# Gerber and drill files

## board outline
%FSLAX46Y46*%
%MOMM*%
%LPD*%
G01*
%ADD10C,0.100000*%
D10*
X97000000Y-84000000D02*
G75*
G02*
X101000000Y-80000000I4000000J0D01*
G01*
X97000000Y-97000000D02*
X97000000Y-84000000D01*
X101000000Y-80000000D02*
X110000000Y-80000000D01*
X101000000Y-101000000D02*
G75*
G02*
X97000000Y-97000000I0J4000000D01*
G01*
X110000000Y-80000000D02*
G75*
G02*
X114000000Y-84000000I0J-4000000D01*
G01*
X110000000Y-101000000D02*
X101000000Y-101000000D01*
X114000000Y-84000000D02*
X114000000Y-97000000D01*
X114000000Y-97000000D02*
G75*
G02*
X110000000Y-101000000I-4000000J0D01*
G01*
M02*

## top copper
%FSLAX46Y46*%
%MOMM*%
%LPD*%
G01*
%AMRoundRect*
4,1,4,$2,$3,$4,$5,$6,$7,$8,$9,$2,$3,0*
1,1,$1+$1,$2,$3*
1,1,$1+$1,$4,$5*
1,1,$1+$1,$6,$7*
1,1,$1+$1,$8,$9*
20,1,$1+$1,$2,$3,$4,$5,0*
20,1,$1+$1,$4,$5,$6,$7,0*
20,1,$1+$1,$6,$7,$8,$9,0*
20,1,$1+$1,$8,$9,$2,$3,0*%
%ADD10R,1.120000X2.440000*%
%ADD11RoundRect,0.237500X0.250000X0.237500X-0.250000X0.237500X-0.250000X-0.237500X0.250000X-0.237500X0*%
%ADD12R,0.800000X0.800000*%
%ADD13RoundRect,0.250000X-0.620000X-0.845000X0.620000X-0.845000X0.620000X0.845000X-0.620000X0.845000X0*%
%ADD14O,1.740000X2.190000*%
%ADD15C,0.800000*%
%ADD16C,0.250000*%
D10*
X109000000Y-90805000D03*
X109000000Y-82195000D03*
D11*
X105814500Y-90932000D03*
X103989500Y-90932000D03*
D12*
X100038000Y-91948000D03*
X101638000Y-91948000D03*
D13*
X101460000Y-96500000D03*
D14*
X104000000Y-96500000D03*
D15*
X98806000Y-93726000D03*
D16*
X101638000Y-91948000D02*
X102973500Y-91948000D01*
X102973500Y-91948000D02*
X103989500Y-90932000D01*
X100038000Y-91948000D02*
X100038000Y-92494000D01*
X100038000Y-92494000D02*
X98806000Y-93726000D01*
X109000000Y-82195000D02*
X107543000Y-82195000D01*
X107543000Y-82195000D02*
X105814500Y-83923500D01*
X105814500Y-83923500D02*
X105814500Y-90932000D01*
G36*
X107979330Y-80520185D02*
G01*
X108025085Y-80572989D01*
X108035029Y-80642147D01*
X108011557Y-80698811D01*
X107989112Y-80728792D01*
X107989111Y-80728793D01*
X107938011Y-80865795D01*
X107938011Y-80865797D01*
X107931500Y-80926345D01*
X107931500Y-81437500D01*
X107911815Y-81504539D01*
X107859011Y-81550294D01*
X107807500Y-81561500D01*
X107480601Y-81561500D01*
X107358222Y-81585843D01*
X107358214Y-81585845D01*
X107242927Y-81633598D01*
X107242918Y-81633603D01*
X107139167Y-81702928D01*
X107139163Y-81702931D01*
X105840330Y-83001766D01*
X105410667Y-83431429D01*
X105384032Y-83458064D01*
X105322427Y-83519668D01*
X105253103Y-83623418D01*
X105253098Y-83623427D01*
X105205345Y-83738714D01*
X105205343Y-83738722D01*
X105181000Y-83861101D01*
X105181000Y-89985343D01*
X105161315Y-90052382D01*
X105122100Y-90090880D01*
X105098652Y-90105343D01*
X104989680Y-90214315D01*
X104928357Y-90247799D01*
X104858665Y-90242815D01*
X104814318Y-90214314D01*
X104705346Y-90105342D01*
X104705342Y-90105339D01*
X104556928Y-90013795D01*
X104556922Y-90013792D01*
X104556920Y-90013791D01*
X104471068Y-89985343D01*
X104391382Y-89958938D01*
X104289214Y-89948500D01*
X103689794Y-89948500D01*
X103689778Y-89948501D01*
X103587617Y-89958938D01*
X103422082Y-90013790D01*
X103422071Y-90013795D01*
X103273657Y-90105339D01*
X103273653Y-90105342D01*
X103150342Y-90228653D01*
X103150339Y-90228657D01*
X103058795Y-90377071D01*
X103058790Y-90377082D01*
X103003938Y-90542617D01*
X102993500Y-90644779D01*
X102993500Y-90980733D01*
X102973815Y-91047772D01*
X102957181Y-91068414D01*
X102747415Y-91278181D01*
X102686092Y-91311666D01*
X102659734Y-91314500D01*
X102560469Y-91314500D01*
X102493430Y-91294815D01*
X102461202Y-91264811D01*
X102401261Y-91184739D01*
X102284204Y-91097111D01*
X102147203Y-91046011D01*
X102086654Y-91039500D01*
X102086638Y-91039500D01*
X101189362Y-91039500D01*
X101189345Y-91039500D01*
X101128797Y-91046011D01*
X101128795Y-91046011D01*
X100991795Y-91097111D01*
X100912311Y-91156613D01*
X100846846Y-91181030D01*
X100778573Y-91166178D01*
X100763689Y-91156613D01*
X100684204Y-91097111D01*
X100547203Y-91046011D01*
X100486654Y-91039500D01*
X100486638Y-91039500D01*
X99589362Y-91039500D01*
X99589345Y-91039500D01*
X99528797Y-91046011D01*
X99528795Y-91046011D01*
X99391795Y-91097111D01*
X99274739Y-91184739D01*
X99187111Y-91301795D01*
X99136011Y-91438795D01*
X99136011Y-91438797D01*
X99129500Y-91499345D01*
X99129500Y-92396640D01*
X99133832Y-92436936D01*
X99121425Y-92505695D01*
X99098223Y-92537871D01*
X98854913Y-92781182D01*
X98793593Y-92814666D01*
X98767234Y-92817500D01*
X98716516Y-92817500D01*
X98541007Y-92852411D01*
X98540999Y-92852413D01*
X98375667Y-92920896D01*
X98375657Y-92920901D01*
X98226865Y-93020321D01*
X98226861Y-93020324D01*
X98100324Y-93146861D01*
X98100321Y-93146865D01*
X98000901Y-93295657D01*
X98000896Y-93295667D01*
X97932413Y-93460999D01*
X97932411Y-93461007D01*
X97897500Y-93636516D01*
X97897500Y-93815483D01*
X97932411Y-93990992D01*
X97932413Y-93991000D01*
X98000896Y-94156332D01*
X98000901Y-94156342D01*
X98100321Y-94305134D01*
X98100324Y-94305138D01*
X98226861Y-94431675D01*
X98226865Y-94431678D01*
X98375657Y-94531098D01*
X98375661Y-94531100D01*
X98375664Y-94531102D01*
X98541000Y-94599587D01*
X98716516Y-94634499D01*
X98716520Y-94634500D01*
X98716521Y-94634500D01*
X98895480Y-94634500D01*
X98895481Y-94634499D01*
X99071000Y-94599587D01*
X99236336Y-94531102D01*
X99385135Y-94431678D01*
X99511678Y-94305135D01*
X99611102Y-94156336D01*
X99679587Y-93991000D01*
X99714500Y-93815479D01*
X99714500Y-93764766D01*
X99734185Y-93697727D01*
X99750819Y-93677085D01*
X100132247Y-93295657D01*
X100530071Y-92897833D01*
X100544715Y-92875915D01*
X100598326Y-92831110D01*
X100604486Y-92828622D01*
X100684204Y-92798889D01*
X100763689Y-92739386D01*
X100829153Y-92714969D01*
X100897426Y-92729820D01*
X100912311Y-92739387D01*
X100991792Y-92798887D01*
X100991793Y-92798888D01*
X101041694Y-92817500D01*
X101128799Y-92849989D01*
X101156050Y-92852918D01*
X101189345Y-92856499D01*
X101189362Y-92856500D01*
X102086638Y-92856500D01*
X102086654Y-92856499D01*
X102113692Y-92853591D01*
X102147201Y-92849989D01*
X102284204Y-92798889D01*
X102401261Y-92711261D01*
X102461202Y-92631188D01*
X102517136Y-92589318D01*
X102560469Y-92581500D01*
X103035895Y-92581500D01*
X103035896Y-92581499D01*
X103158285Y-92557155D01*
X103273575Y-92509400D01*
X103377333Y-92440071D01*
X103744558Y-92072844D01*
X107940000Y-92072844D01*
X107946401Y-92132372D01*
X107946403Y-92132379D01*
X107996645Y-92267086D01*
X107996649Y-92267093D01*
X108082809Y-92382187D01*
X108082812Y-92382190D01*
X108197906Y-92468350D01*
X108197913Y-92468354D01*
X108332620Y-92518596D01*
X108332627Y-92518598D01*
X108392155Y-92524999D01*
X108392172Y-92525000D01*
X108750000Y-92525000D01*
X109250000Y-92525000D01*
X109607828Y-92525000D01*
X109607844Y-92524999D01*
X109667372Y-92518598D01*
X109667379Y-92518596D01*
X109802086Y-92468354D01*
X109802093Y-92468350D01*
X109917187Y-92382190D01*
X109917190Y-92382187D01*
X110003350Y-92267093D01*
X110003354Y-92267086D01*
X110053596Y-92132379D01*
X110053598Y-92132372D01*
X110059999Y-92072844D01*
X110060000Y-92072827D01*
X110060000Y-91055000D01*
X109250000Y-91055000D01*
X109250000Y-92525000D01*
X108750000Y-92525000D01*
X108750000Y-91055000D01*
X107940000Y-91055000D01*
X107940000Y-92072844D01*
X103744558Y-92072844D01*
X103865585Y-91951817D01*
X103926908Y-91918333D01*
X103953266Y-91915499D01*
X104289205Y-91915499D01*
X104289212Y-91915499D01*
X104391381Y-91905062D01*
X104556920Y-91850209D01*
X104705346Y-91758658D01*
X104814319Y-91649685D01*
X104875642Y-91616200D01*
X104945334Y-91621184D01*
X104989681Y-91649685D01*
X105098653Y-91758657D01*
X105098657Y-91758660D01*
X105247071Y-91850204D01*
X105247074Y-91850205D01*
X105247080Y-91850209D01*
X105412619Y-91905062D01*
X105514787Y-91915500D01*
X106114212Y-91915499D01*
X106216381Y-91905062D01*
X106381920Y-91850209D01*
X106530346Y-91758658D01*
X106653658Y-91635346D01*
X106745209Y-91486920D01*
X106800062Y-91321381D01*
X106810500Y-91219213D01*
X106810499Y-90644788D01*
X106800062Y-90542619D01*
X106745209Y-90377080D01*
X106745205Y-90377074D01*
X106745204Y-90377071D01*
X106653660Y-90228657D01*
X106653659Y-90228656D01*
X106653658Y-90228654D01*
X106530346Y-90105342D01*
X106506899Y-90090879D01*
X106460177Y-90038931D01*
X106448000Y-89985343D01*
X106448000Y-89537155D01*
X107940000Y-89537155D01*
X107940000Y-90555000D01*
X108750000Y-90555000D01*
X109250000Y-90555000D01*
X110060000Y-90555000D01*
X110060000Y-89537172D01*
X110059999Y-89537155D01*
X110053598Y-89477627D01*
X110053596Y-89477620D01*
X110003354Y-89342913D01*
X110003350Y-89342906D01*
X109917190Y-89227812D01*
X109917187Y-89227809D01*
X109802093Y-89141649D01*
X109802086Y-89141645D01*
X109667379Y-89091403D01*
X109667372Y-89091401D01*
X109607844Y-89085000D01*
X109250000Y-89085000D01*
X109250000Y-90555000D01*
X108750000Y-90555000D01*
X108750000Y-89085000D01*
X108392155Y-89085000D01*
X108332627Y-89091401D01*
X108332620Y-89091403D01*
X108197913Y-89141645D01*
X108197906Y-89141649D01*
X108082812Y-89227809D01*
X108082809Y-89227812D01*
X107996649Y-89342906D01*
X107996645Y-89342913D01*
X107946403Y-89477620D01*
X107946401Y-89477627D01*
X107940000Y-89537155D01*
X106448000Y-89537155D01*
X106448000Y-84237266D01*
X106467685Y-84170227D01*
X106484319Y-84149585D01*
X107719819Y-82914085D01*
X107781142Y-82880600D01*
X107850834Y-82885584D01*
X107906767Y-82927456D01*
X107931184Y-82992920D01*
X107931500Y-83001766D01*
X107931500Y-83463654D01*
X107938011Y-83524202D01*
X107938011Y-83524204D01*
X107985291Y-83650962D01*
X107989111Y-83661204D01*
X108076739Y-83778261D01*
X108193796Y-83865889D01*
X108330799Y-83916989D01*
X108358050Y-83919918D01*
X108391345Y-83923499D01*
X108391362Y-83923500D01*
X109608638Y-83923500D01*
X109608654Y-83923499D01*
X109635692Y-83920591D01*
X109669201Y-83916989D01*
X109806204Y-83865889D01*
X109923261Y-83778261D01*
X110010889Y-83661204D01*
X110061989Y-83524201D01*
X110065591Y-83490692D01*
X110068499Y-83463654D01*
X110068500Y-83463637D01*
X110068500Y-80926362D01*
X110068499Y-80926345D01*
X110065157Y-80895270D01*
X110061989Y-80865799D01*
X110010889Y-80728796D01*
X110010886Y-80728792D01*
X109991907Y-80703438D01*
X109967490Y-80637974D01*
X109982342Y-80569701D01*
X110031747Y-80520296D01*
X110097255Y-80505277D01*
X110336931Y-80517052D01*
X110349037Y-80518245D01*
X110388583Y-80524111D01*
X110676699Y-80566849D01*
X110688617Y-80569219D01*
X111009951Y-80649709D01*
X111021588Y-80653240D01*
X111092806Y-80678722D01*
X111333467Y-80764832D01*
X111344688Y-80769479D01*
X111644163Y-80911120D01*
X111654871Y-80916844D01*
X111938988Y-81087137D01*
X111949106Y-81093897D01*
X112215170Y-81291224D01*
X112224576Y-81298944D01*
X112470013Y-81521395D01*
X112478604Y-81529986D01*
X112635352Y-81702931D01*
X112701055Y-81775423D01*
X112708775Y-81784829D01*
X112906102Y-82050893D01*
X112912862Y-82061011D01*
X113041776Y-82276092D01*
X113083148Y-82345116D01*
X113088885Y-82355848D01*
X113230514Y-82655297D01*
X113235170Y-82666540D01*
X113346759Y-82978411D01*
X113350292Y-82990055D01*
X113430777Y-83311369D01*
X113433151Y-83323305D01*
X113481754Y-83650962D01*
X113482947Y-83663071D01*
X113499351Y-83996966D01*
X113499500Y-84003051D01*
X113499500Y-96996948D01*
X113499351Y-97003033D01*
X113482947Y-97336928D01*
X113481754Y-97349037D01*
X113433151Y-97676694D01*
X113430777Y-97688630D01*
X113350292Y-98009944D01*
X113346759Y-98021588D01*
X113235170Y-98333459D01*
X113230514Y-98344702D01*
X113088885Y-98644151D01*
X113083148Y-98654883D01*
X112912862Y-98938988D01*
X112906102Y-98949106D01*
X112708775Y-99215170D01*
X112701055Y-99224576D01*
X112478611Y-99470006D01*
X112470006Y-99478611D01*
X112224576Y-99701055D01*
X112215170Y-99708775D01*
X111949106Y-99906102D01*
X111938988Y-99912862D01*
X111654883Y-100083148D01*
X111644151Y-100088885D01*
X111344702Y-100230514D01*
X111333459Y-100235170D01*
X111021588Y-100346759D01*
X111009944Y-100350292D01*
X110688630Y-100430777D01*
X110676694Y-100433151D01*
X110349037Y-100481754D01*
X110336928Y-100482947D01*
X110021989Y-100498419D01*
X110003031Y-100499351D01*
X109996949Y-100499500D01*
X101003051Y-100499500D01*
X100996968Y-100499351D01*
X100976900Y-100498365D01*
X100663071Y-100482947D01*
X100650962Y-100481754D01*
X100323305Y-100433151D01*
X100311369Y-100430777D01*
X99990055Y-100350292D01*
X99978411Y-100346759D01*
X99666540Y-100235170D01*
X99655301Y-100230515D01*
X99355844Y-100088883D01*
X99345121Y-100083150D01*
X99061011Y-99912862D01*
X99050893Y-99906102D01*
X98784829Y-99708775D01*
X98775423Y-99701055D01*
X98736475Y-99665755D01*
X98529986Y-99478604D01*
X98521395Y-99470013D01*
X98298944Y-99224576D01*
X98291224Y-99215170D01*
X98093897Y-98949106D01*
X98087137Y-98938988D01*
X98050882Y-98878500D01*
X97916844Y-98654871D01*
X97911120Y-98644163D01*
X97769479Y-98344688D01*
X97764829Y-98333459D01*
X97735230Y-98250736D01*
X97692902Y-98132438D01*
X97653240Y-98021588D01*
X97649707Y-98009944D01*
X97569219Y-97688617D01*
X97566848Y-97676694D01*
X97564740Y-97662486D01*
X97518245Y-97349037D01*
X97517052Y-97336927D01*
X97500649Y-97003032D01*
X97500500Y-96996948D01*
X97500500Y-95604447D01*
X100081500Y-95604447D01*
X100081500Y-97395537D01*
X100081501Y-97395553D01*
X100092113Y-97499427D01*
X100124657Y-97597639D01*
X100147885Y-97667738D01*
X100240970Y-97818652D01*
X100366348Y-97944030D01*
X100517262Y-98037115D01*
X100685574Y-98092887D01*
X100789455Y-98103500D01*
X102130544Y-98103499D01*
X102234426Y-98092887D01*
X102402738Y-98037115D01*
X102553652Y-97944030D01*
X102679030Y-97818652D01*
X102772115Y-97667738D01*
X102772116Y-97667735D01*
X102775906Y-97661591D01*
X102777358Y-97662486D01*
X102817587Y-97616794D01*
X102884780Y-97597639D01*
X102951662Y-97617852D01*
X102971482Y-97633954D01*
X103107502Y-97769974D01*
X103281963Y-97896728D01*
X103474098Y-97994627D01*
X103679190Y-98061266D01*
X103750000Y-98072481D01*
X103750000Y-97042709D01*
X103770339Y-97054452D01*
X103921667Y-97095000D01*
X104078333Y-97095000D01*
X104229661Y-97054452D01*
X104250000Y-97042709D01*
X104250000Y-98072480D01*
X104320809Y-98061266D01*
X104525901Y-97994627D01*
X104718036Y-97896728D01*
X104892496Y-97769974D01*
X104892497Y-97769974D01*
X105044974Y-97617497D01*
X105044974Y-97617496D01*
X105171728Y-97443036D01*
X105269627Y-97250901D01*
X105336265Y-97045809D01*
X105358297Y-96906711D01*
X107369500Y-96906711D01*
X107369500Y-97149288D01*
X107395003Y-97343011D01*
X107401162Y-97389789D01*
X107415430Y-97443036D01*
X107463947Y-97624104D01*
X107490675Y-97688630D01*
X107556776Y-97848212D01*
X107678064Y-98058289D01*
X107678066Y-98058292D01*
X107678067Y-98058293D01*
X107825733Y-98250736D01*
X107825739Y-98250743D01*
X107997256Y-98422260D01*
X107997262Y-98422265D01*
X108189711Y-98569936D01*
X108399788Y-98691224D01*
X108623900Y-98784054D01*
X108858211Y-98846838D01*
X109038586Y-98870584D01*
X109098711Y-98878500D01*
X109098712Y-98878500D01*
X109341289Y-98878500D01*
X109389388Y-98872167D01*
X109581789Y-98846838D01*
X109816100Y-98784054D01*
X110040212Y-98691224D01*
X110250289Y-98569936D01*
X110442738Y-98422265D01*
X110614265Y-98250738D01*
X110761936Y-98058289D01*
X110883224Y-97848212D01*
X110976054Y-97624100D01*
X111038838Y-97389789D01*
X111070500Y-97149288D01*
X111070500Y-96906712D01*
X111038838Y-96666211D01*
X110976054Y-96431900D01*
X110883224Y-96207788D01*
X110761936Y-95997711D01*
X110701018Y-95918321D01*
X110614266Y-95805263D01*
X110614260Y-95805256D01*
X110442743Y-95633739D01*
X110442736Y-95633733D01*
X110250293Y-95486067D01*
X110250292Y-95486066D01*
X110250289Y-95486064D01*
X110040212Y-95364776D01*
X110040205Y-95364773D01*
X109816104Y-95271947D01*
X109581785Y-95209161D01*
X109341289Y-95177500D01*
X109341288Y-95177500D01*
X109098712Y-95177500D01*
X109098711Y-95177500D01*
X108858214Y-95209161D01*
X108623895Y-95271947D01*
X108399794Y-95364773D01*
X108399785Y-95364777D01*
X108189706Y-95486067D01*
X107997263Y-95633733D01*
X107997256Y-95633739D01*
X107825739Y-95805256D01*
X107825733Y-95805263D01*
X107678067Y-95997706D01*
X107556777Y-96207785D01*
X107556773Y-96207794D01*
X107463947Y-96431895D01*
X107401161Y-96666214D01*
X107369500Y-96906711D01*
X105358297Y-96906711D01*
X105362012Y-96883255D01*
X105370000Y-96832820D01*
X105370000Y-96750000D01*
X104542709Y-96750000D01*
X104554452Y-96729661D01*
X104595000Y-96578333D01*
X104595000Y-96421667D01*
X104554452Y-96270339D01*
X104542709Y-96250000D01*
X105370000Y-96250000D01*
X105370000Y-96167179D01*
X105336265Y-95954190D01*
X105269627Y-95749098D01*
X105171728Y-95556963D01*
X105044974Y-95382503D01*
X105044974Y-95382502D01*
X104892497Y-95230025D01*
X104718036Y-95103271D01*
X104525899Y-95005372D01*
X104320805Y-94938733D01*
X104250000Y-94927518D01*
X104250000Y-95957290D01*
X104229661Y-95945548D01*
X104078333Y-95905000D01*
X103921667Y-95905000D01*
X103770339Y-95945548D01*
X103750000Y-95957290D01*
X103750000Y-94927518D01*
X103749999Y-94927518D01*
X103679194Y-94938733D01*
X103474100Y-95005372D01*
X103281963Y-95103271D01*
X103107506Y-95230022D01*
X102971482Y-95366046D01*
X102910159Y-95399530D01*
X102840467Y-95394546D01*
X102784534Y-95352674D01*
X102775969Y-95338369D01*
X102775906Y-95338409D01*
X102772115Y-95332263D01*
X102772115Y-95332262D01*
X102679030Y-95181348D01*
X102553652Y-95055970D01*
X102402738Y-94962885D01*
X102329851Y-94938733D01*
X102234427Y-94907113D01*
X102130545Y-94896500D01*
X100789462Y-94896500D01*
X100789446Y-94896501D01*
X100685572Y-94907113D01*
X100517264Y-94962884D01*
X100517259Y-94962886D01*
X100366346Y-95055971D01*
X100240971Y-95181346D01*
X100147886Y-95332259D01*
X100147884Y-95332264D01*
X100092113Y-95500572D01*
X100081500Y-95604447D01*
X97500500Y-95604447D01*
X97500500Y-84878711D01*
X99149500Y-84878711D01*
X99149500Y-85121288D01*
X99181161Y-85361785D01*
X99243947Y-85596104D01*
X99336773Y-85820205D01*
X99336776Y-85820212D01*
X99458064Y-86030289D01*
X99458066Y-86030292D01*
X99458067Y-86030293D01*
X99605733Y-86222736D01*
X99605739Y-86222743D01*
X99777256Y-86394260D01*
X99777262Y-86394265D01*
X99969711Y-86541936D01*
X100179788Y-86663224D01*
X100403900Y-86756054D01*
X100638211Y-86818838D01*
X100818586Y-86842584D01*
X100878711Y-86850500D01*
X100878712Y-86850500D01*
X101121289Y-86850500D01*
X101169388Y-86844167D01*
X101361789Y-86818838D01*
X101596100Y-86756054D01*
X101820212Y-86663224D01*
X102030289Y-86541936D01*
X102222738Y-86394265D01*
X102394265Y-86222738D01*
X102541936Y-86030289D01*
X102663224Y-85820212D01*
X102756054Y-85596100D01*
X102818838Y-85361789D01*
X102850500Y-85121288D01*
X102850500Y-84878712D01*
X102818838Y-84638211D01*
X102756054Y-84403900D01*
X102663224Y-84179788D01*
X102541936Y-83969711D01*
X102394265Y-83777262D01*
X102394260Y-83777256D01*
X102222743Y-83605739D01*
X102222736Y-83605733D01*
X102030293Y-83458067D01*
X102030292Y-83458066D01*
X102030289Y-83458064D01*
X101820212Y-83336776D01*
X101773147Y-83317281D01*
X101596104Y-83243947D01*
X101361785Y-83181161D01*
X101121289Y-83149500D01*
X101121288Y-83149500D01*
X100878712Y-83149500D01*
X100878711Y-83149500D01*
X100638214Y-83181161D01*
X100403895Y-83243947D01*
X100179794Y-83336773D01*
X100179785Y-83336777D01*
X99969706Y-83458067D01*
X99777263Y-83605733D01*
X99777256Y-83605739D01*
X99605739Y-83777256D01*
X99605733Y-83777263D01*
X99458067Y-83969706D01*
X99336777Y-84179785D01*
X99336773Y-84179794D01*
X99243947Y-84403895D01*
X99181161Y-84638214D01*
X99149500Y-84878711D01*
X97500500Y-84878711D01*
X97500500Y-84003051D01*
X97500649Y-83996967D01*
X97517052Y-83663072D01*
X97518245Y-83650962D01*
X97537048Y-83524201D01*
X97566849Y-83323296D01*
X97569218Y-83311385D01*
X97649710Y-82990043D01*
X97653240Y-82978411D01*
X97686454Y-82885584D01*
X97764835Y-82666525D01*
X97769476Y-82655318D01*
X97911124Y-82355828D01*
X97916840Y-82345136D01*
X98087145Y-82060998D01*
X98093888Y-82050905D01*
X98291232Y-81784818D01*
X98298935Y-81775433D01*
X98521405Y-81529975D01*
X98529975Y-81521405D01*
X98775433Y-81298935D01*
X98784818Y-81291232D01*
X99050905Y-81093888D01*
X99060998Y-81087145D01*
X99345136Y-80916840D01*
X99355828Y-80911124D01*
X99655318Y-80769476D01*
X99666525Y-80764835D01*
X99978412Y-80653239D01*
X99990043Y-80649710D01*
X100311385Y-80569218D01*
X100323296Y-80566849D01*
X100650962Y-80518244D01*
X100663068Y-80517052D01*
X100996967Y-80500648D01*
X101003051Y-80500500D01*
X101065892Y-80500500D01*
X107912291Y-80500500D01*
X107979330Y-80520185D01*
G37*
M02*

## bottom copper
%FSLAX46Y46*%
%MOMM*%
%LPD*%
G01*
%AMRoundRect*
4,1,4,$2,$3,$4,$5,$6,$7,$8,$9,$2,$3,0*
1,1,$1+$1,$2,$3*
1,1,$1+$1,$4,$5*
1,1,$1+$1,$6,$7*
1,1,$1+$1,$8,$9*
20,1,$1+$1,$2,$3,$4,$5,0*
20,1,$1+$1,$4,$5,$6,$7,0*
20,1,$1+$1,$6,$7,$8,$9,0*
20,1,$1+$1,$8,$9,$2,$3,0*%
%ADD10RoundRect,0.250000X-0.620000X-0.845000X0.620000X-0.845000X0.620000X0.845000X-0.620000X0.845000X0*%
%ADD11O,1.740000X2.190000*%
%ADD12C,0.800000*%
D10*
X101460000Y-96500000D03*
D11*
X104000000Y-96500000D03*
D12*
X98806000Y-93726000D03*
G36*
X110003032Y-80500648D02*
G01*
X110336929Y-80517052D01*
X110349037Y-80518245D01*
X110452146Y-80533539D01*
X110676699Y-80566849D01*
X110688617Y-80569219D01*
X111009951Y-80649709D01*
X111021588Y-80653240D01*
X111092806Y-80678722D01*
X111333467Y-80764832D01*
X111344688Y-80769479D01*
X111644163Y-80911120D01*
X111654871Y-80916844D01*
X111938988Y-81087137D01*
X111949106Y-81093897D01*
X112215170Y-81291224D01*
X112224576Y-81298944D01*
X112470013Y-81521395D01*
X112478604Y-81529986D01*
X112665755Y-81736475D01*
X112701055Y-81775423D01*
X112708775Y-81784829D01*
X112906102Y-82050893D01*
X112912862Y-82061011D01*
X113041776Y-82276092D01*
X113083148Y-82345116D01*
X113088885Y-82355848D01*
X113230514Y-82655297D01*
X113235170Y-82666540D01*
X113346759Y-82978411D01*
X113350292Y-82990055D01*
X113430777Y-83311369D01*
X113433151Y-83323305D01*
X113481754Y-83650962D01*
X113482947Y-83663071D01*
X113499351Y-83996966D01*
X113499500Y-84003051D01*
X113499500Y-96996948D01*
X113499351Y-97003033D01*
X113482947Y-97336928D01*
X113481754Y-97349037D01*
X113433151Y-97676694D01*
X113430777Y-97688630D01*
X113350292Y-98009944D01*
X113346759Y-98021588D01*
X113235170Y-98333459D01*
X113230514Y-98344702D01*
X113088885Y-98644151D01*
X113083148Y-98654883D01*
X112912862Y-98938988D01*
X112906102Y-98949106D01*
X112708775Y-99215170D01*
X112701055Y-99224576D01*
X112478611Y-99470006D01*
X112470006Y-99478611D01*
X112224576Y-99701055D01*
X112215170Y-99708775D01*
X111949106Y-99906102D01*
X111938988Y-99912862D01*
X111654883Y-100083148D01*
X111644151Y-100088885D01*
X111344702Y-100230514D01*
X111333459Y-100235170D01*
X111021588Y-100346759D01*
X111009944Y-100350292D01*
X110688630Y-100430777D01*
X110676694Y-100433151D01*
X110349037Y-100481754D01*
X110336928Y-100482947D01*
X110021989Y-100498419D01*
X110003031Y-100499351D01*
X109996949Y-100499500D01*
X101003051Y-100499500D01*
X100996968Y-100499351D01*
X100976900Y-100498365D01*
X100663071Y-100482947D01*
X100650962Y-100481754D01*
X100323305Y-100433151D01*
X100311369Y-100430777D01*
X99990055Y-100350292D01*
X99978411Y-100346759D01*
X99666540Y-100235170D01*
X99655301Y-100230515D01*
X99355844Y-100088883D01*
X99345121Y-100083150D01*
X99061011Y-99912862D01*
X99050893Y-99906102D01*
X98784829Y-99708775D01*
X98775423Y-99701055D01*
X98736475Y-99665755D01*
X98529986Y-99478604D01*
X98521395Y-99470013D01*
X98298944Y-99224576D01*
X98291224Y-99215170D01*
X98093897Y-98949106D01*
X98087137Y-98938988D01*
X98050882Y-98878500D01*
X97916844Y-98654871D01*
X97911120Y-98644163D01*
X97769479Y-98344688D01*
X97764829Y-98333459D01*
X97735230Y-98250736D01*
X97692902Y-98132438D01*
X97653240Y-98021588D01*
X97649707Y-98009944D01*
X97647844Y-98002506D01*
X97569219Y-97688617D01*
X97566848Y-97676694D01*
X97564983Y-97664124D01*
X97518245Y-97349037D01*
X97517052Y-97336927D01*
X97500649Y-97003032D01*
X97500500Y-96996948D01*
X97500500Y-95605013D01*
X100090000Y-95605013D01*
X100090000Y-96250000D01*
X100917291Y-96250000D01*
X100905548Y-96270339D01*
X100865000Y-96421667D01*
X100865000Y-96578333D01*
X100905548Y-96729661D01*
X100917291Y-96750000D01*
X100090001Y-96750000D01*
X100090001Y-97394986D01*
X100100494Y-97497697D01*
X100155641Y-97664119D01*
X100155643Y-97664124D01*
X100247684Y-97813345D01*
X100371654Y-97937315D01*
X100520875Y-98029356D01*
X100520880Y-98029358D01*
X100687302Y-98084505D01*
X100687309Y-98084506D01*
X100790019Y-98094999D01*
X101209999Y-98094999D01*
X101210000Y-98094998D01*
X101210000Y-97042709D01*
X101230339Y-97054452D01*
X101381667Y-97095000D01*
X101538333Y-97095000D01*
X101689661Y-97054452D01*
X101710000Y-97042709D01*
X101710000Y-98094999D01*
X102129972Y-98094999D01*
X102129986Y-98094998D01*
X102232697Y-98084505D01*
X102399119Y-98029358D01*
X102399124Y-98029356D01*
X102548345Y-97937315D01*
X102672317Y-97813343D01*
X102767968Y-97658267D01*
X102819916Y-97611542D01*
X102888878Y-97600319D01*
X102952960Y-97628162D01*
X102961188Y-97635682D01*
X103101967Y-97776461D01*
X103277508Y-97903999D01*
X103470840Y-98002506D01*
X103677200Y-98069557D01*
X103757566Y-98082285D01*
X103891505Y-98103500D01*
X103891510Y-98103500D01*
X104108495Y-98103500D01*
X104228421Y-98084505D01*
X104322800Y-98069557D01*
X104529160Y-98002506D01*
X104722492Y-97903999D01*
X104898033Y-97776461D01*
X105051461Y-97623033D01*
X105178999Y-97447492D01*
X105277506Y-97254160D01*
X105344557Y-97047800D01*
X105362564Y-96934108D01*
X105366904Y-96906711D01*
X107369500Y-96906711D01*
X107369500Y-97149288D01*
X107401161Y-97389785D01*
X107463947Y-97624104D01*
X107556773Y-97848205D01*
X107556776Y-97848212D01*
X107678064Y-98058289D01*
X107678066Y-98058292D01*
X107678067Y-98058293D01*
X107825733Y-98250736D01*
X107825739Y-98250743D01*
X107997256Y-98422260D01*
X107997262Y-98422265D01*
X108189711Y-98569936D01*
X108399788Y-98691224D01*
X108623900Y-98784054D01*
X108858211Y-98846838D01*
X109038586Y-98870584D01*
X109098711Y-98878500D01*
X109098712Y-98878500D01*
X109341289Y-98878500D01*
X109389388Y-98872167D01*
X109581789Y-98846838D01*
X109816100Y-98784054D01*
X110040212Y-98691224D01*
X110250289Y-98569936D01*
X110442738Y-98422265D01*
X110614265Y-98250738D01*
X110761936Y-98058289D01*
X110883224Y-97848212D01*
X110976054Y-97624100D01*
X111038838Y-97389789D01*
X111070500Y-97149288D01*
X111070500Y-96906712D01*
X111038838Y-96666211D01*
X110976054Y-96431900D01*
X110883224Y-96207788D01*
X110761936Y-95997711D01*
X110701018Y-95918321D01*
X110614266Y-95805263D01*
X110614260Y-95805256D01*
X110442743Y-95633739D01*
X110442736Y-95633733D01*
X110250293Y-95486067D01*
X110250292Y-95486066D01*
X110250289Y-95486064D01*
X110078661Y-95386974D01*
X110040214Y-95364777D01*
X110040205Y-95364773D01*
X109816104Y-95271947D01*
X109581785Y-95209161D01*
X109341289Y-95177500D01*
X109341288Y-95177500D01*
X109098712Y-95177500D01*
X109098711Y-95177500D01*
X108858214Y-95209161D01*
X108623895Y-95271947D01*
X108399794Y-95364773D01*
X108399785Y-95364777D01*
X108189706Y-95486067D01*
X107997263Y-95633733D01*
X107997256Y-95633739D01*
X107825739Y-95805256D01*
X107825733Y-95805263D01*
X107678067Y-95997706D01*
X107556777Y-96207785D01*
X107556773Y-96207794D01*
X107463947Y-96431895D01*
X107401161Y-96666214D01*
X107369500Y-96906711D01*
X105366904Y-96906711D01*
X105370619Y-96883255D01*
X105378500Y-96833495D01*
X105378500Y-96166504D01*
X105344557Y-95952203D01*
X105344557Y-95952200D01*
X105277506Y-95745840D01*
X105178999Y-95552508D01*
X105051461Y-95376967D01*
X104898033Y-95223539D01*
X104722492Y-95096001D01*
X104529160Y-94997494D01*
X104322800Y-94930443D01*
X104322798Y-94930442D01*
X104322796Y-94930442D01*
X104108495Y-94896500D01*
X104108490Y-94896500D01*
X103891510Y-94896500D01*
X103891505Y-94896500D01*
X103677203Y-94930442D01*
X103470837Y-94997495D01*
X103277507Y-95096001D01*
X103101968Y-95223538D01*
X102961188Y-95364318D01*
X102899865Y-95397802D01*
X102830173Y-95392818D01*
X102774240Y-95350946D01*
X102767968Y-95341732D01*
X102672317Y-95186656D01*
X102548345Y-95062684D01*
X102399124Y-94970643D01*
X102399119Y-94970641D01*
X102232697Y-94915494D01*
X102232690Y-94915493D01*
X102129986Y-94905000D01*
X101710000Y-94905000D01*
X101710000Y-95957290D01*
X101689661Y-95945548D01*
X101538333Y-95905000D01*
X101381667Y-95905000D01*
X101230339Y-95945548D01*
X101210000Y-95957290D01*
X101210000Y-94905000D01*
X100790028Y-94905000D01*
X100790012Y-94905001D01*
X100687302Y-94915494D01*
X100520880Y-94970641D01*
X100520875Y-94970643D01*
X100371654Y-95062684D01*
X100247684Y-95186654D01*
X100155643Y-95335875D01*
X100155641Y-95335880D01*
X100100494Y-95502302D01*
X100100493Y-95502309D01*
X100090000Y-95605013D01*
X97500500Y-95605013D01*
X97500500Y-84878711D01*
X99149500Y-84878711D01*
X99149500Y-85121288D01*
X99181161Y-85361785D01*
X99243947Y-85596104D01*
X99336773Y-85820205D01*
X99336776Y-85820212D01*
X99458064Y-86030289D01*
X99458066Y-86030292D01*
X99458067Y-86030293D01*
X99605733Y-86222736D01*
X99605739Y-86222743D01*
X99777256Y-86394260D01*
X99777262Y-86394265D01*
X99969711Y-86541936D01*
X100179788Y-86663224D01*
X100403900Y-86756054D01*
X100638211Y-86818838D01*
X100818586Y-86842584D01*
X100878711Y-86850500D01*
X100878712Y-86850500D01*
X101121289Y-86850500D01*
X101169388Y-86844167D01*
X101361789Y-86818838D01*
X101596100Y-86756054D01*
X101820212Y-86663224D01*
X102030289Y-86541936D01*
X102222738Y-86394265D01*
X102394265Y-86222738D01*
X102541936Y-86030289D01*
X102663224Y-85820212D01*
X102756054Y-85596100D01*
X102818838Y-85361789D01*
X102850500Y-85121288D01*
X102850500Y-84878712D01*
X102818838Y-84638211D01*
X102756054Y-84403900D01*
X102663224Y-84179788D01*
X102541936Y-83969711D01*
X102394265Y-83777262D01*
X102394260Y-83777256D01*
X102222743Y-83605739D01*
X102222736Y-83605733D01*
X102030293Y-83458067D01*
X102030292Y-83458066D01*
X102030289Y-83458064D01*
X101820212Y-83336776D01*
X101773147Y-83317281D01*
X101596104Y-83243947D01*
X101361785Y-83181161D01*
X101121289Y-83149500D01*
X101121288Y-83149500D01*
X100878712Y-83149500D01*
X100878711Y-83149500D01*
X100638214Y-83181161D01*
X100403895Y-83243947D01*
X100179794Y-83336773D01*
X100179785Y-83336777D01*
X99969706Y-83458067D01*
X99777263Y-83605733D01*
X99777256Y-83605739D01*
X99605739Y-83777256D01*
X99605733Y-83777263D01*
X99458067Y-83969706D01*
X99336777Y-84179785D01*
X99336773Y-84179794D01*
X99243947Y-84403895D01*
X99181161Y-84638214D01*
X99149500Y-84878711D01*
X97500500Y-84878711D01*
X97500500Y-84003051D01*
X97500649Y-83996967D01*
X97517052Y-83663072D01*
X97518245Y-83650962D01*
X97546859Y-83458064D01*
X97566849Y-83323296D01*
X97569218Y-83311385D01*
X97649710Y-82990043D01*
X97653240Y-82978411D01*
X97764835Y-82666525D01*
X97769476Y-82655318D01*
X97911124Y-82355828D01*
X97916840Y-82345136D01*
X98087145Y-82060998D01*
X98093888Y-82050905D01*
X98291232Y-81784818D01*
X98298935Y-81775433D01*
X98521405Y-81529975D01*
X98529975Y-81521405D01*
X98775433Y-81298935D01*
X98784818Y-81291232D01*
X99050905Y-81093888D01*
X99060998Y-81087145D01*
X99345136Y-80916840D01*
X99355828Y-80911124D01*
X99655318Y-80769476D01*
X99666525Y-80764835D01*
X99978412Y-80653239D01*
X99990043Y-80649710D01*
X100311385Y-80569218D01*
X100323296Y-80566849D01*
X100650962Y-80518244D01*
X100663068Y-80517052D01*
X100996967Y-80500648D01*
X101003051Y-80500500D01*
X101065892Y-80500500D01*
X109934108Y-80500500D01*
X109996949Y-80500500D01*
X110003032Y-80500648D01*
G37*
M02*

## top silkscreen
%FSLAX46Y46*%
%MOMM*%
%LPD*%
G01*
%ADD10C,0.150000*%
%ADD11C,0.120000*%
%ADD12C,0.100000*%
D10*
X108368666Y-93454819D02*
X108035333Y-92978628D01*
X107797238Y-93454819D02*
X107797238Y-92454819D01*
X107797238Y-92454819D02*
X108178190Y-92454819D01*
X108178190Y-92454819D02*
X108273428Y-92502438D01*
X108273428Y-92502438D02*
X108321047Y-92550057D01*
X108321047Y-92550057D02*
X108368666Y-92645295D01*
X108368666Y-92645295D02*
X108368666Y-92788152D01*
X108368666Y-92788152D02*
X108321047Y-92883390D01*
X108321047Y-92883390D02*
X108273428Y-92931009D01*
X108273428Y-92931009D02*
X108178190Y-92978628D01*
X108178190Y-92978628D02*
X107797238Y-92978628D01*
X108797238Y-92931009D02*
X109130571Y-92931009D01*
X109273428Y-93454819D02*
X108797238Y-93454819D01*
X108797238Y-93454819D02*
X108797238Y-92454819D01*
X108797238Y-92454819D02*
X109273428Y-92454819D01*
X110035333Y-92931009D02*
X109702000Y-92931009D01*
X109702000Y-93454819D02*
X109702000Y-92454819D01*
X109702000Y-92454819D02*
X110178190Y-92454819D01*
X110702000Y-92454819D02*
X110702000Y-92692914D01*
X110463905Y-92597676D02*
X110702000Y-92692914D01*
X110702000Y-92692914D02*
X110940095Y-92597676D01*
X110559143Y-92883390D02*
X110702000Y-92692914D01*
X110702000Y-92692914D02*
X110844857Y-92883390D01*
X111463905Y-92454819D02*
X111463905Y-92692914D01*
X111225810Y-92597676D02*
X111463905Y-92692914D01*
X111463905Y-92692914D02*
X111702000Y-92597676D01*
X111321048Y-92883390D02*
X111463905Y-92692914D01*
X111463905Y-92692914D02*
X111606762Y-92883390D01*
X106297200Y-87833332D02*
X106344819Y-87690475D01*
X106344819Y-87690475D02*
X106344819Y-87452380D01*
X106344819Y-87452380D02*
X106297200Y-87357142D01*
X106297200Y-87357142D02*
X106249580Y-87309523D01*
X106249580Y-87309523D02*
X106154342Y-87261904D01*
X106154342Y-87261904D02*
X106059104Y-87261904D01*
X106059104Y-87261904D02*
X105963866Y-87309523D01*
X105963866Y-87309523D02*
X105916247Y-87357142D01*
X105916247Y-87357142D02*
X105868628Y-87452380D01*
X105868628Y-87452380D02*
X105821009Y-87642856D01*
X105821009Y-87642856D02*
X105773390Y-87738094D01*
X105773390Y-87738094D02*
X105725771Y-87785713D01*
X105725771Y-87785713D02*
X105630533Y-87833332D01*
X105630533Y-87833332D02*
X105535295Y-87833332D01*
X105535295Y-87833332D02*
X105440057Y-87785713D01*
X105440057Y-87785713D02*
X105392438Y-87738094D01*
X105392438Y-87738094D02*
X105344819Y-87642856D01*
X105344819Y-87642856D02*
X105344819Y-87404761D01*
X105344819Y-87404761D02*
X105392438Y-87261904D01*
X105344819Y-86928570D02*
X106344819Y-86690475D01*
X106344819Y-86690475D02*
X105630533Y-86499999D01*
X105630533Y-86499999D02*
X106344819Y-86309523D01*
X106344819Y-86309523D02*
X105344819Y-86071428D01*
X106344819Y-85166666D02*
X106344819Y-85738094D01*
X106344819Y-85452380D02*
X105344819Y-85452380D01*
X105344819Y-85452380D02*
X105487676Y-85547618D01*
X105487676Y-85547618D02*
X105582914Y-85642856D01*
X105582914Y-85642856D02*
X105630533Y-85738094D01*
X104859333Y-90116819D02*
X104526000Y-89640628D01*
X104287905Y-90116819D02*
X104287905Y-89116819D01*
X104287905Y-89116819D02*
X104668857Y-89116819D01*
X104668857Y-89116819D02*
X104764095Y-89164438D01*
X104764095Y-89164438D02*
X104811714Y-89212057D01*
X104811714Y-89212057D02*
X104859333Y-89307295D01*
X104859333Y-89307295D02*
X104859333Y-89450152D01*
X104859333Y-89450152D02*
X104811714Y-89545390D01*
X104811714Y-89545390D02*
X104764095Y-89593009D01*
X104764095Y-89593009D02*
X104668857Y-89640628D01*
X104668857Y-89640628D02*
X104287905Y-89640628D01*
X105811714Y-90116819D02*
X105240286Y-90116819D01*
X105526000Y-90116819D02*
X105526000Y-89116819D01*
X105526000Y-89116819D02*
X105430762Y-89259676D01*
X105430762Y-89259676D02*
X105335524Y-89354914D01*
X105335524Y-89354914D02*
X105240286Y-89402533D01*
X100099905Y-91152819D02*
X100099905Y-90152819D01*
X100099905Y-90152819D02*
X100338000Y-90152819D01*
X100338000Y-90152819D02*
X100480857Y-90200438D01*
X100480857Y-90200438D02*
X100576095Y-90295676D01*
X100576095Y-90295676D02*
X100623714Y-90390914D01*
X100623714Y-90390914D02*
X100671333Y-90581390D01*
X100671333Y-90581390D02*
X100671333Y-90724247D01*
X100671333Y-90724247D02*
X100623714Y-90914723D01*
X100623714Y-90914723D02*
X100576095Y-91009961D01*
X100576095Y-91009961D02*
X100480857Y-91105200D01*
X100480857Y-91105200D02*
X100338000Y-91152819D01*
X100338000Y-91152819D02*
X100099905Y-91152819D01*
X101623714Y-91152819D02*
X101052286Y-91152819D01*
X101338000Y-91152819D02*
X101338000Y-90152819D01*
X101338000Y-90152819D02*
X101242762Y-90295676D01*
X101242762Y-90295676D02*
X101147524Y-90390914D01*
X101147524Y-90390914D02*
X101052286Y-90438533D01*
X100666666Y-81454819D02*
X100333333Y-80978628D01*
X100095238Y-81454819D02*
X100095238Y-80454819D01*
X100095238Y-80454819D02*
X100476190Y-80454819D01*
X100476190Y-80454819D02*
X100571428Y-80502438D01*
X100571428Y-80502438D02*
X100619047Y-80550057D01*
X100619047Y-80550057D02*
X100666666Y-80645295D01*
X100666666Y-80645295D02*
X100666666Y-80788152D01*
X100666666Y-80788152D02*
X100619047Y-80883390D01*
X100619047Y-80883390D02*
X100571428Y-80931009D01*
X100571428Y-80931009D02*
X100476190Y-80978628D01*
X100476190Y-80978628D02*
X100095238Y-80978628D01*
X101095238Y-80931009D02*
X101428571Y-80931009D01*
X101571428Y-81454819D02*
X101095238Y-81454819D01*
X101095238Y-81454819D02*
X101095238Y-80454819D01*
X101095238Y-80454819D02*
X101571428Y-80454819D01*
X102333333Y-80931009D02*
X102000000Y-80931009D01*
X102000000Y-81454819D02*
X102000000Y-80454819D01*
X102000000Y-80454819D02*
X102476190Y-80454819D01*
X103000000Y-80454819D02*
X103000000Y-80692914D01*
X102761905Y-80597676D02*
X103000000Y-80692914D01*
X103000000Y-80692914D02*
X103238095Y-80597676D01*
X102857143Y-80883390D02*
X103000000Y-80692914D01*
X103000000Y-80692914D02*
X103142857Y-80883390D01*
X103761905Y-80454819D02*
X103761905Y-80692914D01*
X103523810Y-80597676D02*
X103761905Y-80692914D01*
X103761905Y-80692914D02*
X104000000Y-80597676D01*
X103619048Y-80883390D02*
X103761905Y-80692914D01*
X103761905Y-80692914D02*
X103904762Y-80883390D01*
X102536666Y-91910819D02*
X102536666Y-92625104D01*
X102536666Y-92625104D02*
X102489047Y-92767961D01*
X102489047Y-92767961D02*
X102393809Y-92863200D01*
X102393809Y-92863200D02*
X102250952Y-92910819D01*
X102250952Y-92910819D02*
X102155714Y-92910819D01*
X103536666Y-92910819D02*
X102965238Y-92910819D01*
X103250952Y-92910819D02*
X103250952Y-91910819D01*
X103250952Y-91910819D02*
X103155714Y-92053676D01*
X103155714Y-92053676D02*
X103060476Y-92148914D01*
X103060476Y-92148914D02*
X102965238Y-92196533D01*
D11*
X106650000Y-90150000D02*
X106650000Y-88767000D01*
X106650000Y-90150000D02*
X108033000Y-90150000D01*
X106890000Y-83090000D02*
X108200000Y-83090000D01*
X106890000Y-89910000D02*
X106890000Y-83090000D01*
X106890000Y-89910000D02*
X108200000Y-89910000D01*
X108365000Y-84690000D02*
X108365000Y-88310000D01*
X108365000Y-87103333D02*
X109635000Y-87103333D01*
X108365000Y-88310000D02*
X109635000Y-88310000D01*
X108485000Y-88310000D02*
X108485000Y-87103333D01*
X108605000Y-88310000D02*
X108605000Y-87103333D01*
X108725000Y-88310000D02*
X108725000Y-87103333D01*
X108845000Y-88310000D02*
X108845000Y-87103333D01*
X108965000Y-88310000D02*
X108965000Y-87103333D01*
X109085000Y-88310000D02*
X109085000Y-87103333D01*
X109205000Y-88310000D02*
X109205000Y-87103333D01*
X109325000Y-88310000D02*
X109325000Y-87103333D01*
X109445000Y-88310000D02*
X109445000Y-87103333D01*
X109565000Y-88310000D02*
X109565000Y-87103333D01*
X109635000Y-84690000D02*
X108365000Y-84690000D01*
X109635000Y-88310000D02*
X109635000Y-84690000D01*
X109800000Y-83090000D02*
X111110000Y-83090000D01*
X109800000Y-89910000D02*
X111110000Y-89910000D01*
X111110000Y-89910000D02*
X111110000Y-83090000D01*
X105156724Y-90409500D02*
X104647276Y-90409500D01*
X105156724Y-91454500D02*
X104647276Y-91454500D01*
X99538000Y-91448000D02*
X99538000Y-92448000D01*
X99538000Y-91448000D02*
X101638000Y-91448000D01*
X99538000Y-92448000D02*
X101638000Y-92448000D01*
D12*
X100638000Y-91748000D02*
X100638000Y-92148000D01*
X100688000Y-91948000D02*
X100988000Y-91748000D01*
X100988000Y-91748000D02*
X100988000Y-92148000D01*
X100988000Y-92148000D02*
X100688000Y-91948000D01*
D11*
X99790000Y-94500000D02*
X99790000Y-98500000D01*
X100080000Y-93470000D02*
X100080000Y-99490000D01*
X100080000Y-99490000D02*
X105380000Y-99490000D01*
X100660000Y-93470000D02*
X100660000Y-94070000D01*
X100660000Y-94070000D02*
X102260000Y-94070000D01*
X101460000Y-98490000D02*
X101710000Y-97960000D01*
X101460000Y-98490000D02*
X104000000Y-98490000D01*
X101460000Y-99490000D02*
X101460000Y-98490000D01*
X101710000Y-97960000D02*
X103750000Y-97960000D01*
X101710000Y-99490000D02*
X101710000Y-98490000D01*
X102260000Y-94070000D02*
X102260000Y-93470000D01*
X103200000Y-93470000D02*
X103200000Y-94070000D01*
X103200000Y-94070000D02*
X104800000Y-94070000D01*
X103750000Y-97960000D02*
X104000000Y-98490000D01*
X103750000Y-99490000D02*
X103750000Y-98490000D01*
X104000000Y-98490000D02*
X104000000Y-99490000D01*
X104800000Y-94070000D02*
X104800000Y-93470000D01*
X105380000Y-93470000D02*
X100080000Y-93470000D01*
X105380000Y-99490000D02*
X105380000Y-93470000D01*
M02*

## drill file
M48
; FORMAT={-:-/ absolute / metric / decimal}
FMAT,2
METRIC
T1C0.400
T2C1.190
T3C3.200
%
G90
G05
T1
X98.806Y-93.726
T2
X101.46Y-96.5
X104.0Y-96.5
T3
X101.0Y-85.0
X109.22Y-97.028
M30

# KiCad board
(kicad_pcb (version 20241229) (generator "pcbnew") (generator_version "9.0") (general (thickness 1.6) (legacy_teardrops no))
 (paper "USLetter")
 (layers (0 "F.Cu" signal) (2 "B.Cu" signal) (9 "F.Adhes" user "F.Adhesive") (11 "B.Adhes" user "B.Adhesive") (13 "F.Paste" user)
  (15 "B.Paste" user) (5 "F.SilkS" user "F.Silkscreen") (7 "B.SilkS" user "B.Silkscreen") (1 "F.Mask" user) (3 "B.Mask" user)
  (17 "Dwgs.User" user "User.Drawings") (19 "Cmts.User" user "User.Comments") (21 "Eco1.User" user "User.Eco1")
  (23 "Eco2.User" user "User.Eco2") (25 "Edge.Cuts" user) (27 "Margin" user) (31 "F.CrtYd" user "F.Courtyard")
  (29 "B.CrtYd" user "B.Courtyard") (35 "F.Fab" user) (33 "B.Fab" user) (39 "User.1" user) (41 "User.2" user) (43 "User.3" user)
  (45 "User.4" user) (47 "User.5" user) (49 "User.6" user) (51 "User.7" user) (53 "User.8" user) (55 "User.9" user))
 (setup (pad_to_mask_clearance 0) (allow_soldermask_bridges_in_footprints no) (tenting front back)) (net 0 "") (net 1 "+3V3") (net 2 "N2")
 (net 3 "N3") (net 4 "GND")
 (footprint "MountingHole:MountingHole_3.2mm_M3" (layer "F.Cu") (at 109.22 97.028)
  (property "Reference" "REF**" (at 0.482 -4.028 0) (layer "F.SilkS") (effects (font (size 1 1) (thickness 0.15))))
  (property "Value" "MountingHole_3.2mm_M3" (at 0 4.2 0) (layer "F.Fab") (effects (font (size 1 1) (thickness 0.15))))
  (pad "" np_thru_hole circle (at 0 0) (size 3.2 3.2) (drill 3.2) (layers "*.Cu" "*.Mask")))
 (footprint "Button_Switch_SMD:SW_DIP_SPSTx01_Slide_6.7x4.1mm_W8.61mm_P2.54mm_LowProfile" (layer "F.Cu") (at 109 86.5 90)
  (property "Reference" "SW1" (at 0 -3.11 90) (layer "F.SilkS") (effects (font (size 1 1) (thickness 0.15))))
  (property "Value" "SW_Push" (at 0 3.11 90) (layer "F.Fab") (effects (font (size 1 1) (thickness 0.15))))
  (fp_line (start -3.65 -2.35) (end -2.267 -2.35) (stroke (width 0.12) (type solid)) (layer "F.SilkS"))
  (fp_line (start -3.65 -2.35) (end -3.65 -0.967) (stroke (width 0.12) (type solid)) (layer "F.SilkS"))
  (fp_line (start 3.41 -2.11) (end 3.41 -0.8) (stroke (width 0.12) (type solid)) (layer "F.SilkS"))
  (fp_line (start -3.41 -2.11) (end 3.41 -2.11) (stroke (width 0.12) (type solid)) (layer "F.SilkS"))
  (fp_line (start -3.41 -2.11) (end -3.41 -0.8) (stroke (width 0.12) (type solid)) (layer "F.SilkS"))
  (fp_line (start 1.81 -0.635) (end -1.81 -0.635) (stroke (width 0.12) (type solid)) (layer "F.SilkS"))
  (fp_line (start -0.603333 -0.635) (end -0.603333 0.635) (stroke (width 0.12) (type solid)) (layer "F.SilkS"))
  (fp_line (start -1.81 -0.635) (end -1.81 0.635) (stroke (width 0.12) (type solid)) (layer "F.SilkS"))
  (fp_line (start -1.81 -0.515) (end -0.603333 -0.515) (stroke (width 0.12) (type solid)) (layer "F.SilkS"))
  (fp_line (start -1.81 -0.395) (end -0.603333 -0.395) (stroke (width 0.12) (type solid)) (layer "F.SilkS"))
  (fp_line (start -1.81 -0.275) (end -0.603333 -0.275) (stroke (width 0.12) (type solid)) (layer "F.SilkS"))
  (fp_line (start -1.81 -0.155) (end -0.603333 -0.155) (stroke (width 0.12) (type solid)) (layer "F.SilkS"))
  (fp_line (start -1.81 -0.035) (end -0.603333 -0.035) (stroke (width 0.12) (type solid)) (layer "F.SilkS"))
  (fp_line (start -1.81 0.085) (end -0.603333 0.085) (stroke (width 0.12) (type solid)) (layer "F.SilkS"))
  (fp_line (start -1.81 0.205) (end -0.603333 0.205) (stroke (width 0.12) (type solid)) (layer "F.SilkS"))
  (fp_line (start -1.81 0.325) (end -0.603333 0.325) (stroke (width 0.12) (type solid)) (layer "F.SilkS"))
  (fp_line (start -1.81 0.445) (end -0.603333 0.445) (stroke (width 0.12) (type solid)) (layer "F.SilkS"))
  (fp_line (start -1.81 0.565) (end -0.603333 0.565) (stroke (width 0.12) (type solid)) (layer "F.SilkS"))
  (fp_line (start 1.81 0.635) (end 1.81 -0.635) (stroke (width 0.12) (type solid)) (layer "F.SilkS"))
  (fp_line (start -1.81 0.635) (end 1.81 0.635) (stroke (width 0.12) (type solid)) (layer "F.SilkS"))
  (fp_line (start 3.41 0.8) (end 3.41 2.11) (stroke (width 0.12) (type solid)) (layer "F.SilkS"))
  (fp_line (start -3.41 0.8) (end -3.41 2.11) (stroke (width 0.12) (type solid)) (layer "F.SilkS"))
  (fp_line (start -3.41 2.11) (end 3.41 2.11) (stroke (width 0.12) (type solid)) (layer "F.SilkS"))
  (pad "1" smd rect (at -4.305 0 90) (size 2.44 1.12) (layers "F.Cu" "F.Mask" "F.Paste") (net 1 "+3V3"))
  (pad "2" smd rect (at 4.305 0 90) (size 2.44 1.12) (layers "F.Cu" "F.Mask" "F.Paste") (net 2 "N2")))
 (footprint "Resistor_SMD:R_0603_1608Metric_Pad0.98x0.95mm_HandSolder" (layer "F.Cu") (at 104.902 90.932 180)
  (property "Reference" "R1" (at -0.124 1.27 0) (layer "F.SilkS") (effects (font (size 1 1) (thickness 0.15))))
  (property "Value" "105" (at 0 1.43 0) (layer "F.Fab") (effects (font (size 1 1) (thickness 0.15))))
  (fp_line (start -0.254724 0.5225) (end 0.254724 0.5225) (stroke (width 0.12) (type solid)) (layer "F.SilkS"))
  (fp_line (start -0.254724 -0.5225) (end 0.254724 -0.5225) (stroke (width 0.12) (type solid)) (layer "F.SilkS"))
  (pad "1" smd roundrect (at -0.9125 0 180) (size 0.975 0.95) (layers "F.Cu" "F.Mask" "F.Paste") (roundrect_rratio 0.25) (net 2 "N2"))
  (pad "2" smd roundrect (at 0.9125 0 180) (size 0.975 0.95) (layers "F.Cu" "F.Mask" "F.Paste") (roundrect_rratio 0.25) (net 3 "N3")))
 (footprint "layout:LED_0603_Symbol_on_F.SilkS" (layer "F.Cu") (at 100.838 91.948)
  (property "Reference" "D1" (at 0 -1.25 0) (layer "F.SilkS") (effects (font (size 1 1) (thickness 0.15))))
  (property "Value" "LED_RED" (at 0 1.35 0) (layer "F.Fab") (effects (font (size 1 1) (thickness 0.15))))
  (fp_line (start -1.3 -0.5) (end -1.3 0.5) (stroke (width 0.12) (type solid)) (layer "F.SilkS"))
  (fp_line (start -1.3 -0.5) (end 0.8 -0.5) (stroke (width 0.12) (type solid)) (layer "F.SilkS"))
  (fp_line (start -1.3 0.5) (end 0.8 0.5) (stroke (width 0.12) (type solid)) (layer "F.SilkS"))
  (fp_line (start -0.2 -0.2) (end -0.2 0.2) (stroke (width 0.1) (type solid)) (layer "F.SilkS"))
  (fp_line (start -0.15 0) (end 0.15 -0.2) (stroke (width 0.1) (type solid)) (layer "F.SilkS"))
  (fp_line (start 0.15 -0.2) (end 0.15 0.2) (stroke (width 0.1) (type solid)) (layer "F.SilkS"))
  (fp_line (start 0.15 0.2) (end -0.15 0) (stroke (width 0.1) (type solid)) (layer "F.SilkS"))
  (pad "1" smd rect (at -0.8 0 180) (size 0.8 0.8) (layers "F.Cu" "F.Mask" "F.Paste") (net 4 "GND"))
  (pad "2" smd rect (at 0.8 0 180) (size 0.8 0.8) (layers "F.Cu" "F.Mask" "F.Paste") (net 3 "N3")))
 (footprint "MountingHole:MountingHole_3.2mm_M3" (layer "F.Cu") (at 101 85)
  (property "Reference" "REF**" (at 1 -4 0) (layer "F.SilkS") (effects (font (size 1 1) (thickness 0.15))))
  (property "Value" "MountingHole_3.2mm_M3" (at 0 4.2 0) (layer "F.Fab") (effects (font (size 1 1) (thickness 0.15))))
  (pad "" np_thru_hole circle (at 0 0) (size 3.2 3.2) (drill 3.2) (layers "*.Cu" "*.Mask")))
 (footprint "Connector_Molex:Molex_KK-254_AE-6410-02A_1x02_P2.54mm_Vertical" (layer "F.Cu") (at 101.46 96.5)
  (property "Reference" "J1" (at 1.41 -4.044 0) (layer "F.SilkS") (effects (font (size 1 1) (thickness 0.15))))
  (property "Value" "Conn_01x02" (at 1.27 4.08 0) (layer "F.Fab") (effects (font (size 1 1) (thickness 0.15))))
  (fp_line (start -1.67 -2) (end -1.67 2) (stroke (width 0.12) (type solid)) (layer "F.SilkS"))
  (fp_line (start -1.38 -3.03) (end -1.38 2.99) (stroke (width 0.12) (type solid)) (layer "F.SilkS"))
  (fp_line (start -1.38 2.99) (end 3.92 2.99) (stroke (width 0.12) (type solid)) (layer "F.SilkS"))
  (fp_line (start -0.8 -3.03) (end -0.8 -2.43) (stroke (width 0.12) (type solid)) (layer "F.SilkS"))
  (fp_line (start -0.8 -2.43) (end 0.8 -2.43) (stroke (width 0.12) (type solid)) (layer "F.SilkS"))
  (fp_line (start 0 1.99) (end 0.25 1.46) (stroke (width 0.12) (type solid)) (layer "F.SilkS"))
  (fp_line (start 0 1.99) (end 2.54 1.99) (stroke (width 0.12) (type solid)) (layer "F.SilkS"))
  (fp_line (start 0 2.99) (end 0 1.99) (stroke (width 0.12) (type solid)) (layer "F.SilkS"))
  (fp_line (start 0.25 1.46) (end 2.29 1.46) (stroke (width 0.12) (type solid)) (layer "F.SilkS"))
  (fp_line (start 0.25 2.99) (end 0.25 1.99) (stroke (width 0.12) (type solid)) (layer "F.SilkS"))
  (fp_line (start 0.8 -2.43) (end 0.8 -3.03) (stroke (width 0.12) (type solid)) (layer "F.SilkS"))
  (fp_line (start 1.74 -3.03) (end 1.74 -2.43) (stroke (width 0.12) (type solid)) (layer "F.SilkS"))
  (fp_line (start 1.74 -2.43) (end 3.34 -2.43) (stroke (width 0.12) (type solid)) (layer "F.SilkS"))
  (fp_line (start 2.29 1.46) (end 2.54 1.99) (stroke (width 0.12) (type solid)) (layer "F.SilkS"))
  (fp_line (start 2.29 2.99) (end 2.29 1.99) (stroke (width 0.12) (type solid)) (layer "F.SilkS"))
  (fp_line (start 2.54 1.99) (end 2.54 2.99) (stroke (width 0.12) (type solid)) (layer "F.SilkS"))
  (fp_line (start 3.34 -2.43) (end 3.34 -3.03) (stroke (width 0.12) (type solid)) (layer "F.SilkS"))
  (fp_line (start 3.92 -3.03) (end -1.38 -3.03) (stroke (width 0.12) (type solid)) (layer "F.SilkS"))
  (fp_line (start 3.92 2.99) (end 3.92 -3.03) (stroke (width 0.12) (type solid)) (layer "F.SilkS"))
  (pad "1" thru_hole roundrect (at 0 0) (size 1.74 2.19) (drill 1.19) (layers "*.Cu" "*.Mask") (remove_unused_layers no)
   (roundrect_rratio 0.143678) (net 4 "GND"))
  (pad "2" thru_hole oval (at 2.54 0) (size 1.74 2.19) (drill 1.19) (layers "*.Cu" "*.Mask") (remove_unused_layers no) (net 1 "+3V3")))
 (gr_arc (start 97 84) (mid 98.171573 81.171573) (end 101 80) (stroke (width 0.1) (type default)) (layer "Edge.Cuts"))
 (gr_line (start 97 97) (end 97 84) (stroke (width 0.1) (type default)) (layer "Edge.Cuts"))
 (gr_line (start 101 80) (end 110 80) (stroke (width 0.1) (type default)) (layer "Edge.Cuts"))
 (gr_arc (start 101 101) (mid 98.171573 99.828427) (end 97 97) (stroke (width 0.1) (type default)) (layer "Edge.Cuts"))
 (gr_arc (start 110 80) (mid 112.828427 81.171573) (end 114 84) (stroke (width 0.1) (type default)) (layer "Edge.Cuts"))
 (gr_line (start 110 101) (end 101 101) (stroke (width 0.1) (type default)) (layer "Edge.Cuts"))
 (gr_line (start 114 84) (end 114 97) (stroke (width 0.1) (type default)) (layer "Edge.Cuts"))
 (gr_arc (start 114 97) (mid 112.828427 99.828427) (end 110 101) (stroke (width 0.1) (type default)) (layer "Edge.Cuts"))
 (segment (start 101.638 91.948) (end 102.9735 91.948) (width 0.25) (layer "F.Cu") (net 3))
 (segment (start 102.9735 91.948) (end 103.9895 90.932) (width 0.25) (layer "F.Cu") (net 3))
 (segment (start 100.038 91.948) (end 100.038 92.494) (width 0.25) (layer "F.Cu") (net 4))
 (segment (start 100.038 92.494) (end 98.806 93.726) (width 0.25) (layer "F.Cu") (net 4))
 (via (at 98.806 93.726) (size 0.8) (drill 0.4) (layers "F.Cu" "B.Cu") (free yes) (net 4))
 (segment (start 109 82.195) (end 107.543 82.195) (width 0.25) (layer "F.Cu") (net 2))
 (segment (start 107.543 82.195) (end 105.8145 83.9235) (width 0.25) (layer "F.Cu") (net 2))
 (segment (start 105.8145 83.9235) (end 105.8145 90.932) (width 0.25) (layer "F.Cu") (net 2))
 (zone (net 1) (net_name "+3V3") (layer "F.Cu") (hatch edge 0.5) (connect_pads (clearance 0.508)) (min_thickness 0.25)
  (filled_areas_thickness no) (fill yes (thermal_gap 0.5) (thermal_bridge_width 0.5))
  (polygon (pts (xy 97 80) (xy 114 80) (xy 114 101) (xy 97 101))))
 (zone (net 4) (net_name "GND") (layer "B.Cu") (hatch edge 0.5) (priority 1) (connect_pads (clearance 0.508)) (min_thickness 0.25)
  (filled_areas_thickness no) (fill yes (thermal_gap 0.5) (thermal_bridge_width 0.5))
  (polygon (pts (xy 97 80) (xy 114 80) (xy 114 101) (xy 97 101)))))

